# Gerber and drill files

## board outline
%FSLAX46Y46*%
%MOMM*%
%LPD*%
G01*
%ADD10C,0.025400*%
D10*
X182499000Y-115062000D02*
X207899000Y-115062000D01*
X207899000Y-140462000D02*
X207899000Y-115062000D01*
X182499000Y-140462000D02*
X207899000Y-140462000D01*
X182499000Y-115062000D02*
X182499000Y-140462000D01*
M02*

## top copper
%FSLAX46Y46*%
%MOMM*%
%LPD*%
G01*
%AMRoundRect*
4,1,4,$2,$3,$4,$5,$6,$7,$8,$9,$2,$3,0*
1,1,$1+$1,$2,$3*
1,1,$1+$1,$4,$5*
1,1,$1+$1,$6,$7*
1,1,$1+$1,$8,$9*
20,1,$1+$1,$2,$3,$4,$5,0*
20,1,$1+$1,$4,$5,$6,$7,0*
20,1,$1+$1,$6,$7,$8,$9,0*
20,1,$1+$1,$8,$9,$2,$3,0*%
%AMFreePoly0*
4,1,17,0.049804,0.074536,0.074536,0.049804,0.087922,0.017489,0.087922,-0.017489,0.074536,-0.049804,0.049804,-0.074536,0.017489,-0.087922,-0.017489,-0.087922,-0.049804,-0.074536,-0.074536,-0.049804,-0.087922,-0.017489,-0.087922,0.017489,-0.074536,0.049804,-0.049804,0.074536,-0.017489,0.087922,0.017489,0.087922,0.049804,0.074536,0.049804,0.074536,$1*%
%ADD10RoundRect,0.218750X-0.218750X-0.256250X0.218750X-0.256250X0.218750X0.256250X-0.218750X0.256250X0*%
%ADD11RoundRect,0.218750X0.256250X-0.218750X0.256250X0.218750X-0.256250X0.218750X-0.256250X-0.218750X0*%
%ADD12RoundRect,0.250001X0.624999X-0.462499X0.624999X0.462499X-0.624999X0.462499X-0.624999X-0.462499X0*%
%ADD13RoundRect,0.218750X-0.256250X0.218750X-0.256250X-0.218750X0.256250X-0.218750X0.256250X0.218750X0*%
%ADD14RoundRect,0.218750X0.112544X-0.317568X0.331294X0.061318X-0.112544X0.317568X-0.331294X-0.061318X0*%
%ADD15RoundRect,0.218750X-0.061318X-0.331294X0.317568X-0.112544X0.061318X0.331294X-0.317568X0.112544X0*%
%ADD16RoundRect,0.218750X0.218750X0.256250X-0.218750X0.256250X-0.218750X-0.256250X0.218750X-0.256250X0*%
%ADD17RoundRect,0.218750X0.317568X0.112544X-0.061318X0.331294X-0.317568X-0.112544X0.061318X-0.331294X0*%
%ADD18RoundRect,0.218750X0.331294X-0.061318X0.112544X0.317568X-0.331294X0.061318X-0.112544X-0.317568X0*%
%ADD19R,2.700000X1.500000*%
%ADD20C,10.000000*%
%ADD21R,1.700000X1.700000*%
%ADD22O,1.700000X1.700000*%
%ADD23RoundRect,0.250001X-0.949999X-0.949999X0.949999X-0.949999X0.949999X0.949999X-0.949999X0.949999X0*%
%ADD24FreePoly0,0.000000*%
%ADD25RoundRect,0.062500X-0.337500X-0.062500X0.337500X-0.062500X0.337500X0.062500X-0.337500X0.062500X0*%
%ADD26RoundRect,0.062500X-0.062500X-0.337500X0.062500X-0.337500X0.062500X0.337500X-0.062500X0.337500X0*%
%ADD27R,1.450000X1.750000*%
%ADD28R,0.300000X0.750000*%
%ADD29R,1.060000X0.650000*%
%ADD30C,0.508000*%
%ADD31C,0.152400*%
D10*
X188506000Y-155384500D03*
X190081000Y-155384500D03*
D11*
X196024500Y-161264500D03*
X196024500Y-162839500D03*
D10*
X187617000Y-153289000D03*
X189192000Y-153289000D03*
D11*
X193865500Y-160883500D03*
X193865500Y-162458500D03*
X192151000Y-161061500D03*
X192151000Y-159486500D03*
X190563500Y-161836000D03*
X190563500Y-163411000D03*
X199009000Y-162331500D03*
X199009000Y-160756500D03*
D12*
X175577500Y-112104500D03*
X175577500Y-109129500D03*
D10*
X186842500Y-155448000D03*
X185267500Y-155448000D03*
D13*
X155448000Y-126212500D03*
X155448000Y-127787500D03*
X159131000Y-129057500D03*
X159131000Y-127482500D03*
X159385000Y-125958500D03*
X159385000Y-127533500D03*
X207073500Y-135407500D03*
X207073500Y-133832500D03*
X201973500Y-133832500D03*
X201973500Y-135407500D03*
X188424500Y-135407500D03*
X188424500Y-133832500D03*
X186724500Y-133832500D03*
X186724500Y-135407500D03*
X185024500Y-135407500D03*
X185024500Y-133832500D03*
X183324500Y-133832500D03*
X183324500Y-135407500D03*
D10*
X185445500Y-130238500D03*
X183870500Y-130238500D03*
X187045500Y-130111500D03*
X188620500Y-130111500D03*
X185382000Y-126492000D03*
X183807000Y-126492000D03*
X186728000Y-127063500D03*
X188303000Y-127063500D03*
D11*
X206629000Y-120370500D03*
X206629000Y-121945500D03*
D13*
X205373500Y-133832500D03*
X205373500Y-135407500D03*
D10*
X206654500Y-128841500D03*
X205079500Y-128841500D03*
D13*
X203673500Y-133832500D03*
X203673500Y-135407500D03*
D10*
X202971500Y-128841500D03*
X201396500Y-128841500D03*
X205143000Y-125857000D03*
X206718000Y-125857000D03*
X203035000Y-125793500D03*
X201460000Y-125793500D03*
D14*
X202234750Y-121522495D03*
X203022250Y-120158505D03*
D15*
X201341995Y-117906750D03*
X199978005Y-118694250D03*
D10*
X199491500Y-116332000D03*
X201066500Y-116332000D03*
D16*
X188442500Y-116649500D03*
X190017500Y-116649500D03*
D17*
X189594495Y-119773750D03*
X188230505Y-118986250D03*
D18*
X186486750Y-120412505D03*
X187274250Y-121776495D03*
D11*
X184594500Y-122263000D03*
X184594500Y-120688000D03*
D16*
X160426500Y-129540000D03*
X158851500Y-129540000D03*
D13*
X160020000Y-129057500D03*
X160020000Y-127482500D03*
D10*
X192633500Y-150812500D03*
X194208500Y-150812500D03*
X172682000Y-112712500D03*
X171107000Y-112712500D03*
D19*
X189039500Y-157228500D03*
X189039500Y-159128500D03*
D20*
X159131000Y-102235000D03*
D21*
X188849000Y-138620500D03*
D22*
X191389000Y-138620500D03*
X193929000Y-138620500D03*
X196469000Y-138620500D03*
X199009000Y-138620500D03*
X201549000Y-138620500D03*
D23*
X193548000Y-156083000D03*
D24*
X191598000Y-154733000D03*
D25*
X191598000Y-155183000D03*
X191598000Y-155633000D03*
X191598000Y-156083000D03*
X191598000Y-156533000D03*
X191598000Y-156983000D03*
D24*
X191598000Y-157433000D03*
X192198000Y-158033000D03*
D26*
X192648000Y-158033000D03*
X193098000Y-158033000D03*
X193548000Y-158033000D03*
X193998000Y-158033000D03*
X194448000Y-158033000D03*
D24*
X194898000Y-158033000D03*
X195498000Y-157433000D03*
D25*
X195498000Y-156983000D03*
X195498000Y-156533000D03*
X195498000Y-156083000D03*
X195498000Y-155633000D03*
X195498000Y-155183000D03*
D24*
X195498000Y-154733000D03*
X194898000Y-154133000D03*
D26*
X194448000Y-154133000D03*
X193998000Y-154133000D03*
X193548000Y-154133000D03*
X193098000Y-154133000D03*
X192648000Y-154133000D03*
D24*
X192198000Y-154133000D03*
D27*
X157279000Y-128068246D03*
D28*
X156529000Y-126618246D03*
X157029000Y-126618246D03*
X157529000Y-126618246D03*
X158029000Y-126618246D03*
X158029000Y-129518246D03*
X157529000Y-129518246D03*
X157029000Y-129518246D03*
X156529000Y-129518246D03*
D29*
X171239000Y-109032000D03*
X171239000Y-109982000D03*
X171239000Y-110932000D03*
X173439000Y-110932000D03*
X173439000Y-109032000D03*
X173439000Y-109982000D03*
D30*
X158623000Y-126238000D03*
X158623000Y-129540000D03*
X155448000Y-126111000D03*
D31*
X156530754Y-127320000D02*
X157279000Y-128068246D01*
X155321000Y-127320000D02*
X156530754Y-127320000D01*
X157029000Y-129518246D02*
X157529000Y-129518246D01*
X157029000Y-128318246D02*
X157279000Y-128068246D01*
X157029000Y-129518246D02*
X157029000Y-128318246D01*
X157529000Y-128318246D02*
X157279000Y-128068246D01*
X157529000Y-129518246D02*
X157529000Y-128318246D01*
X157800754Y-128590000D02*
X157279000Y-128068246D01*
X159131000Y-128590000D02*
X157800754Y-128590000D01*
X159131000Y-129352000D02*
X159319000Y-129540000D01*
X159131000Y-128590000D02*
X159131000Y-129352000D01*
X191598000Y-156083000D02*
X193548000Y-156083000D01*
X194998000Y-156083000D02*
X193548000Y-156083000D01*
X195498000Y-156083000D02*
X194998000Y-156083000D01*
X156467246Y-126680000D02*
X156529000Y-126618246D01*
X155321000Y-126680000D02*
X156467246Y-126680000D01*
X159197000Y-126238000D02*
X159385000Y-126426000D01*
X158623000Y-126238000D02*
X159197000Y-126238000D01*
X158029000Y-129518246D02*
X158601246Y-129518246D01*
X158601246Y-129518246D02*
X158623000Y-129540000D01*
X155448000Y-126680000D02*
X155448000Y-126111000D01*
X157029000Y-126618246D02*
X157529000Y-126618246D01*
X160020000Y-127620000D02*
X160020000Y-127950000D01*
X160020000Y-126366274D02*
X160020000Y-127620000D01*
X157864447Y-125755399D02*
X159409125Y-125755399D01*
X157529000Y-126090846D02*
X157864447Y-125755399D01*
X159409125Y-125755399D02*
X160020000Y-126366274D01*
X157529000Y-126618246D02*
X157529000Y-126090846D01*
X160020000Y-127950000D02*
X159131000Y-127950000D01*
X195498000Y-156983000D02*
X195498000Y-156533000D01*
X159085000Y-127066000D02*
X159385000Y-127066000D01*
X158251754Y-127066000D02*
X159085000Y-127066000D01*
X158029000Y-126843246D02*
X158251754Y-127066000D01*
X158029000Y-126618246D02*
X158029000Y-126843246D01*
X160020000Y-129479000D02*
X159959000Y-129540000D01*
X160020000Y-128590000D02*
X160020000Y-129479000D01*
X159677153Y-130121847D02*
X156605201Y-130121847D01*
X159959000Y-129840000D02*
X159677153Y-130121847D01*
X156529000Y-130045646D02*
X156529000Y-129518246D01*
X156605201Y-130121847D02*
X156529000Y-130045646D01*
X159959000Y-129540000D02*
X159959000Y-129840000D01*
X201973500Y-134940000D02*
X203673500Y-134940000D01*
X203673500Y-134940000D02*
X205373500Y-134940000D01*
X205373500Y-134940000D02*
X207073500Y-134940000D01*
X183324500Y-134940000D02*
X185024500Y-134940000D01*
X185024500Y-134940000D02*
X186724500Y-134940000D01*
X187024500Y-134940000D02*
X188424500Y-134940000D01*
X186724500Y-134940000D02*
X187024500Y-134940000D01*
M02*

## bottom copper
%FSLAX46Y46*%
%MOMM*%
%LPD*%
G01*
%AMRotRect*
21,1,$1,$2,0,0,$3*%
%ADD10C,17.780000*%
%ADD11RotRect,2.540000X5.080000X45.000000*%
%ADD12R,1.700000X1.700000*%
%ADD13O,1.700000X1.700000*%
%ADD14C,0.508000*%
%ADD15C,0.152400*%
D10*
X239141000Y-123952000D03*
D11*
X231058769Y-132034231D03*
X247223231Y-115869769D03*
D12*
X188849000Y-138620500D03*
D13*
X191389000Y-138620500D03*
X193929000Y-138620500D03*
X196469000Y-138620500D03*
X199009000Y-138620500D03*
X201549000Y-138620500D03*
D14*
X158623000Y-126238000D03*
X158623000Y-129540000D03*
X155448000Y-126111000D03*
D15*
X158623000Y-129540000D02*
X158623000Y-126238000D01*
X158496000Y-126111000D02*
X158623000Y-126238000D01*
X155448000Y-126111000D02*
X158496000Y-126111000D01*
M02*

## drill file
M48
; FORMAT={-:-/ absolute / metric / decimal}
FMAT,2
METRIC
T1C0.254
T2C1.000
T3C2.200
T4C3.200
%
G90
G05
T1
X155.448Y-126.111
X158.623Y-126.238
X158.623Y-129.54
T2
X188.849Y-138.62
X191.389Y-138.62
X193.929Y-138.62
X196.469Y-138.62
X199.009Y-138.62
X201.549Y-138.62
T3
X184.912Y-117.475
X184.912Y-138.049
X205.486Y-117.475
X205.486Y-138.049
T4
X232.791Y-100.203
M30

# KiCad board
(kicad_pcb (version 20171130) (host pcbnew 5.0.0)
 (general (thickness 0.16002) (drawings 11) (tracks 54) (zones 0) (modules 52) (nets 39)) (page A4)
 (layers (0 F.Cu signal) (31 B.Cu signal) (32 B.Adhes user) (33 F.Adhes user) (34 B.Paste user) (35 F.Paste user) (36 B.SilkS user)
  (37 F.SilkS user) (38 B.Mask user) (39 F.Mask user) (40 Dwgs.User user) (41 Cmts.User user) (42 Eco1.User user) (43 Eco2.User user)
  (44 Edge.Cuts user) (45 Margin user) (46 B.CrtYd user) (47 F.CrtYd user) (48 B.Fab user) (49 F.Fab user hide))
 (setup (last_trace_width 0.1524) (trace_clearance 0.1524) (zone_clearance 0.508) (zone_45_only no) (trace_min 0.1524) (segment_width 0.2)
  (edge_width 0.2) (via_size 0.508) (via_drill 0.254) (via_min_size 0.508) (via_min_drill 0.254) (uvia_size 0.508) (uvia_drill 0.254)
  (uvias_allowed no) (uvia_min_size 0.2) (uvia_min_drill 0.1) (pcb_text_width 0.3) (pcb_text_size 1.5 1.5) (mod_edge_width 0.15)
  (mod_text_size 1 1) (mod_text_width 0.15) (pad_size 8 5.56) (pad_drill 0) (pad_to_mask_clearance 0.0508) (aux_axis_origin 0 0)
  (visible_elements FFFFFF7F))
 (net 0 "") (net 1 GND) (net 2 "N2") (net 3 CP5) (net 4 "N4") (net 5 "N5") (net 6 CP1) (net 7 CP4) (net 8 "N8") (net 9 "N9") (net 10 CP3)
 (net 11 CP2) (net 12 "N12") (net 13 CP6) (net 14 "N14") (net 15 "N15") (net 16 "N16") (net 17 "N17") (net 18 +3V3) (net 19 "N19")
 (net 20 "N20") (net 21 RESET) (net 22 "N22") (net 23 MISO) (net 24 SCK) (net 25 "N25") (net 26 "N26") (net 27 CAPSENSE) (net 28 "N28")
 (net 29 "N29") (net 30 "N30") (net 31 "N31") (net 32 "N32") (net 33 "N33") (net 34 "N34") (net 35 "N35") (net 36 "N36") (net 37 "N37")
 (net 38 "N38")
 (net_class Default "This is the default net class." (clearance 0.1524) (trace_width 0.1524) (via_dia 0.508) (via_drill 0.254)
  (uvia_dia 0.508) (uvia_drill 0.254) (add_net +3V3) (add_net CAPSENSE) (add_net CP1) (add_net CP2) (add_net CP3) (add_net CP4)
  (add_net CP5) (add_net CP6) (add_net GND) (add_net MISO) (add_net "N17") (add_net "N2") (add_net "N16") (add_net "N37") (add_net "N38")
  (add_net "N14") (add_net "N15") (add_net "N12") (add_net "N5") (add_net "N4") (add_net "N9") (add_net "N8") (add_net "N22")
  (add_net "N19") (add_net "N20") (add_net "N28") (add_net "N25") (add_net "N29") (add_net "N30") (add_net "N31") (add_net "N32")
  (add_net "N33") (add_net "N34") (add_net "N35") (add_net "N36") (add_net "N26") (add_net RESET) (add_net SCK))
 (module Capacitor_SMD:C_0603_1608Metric (layer F.Cu) (at 189.2935 155.3845)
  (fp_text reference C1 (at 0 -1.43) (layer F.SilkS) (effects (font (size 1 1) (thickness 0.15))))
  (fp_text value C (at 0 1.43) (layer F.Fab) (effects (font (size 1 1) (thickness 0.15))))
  (pad 1 smd roundrect (at -0.7875 0) (size 0.875 0.95) (layers F.Cu F.Paste F.Mask) (roundrect_rratio 0.25) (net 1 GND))
  (pad 2 smd roundrect (at 0.7875 0) (size 0.875 0.95) (layers F.Cu F.Paste F.Mask) (roundrect_rratio 0.25) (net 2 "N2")))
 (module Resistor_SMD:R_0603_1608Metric (layer F.Cu) (at 196.0245 162.052 90)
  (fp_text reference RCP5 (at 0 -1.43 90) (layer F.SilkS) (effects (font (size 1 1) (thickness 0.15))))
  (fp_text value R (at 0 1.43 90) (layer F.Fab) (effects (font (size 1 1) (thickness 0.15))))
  (pad 2 smd roundrect (at 0.7875 0 90) (size 0.875 0.95) (layers F.Cu F.Paste F.Mask) (roundrect_rratio 0.25) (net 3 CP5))
  (pad 1 smd roundrect (at -0.7875 0 90) (size 0.875 0.95) (layers F.Cu F.Paste F.Mask) (roundrect_rratio 0.25) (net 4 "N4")))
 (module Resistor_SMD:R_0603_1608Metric (layer F.Cu) (at 188.4045 153.289)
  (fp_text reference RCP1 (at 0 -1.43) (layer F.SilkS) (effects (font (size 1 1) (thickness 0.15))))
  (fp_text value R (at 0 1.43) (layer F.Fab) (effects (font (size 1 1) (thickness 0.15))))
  (pad 1 smd roundrect (at -0.7875 0) (size 0.875 0.95) (layers F.Cu F.Paste F.Mask) (roundrect_rratio 0.25) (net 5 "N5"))
  (pad 2 smd roundrect (at 0.7875 0) (size 0.875 0.95) (layers F.Cu F.Paste F.Mask) (roundrect_rratio 0.25) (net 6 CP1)))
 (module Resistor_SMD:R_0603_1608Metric (layer F.Cu) (at 193.8655 161.671 90)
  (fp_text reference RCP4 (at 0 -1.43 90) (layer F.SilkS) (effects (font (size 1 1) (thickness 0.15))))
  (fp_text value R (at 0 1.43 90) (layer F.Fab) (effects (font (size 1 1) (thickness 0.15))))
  (pad 2 smd roundrect (at 0.7875 0 90) (size 0.875 0.95) (layers F.Cu F.Paste F.Mask) (roundrect_rratio 0.25) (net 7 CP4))
  (pad 1 smd roundrect (at -0.7875 0 90) (size 0.875 0.95) (layers F.Cu F.Paste F.Mask) (roundrect_rratio 0.25) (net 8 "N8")))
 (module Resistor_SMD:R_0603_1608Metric (layer F.Cu) (at 192.151 160.274 90)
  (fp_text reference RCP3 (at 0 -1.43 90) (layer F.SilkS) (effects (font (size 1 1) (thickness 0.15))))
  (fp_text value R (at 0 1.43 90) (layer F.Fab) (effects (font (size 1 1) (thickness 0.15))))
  (pad 1 smd roundrect (at -0.7875 0 90) (size 0.875 0.95) (layers F.Cu F.Paste F.Mask) (roundrect_rratio 0.25) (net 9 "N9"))
  (pad 2 smd roundrect (at 0.7875 0 90) (size 0.875 0.95) (layers F.Cu F.Paste F.Mask) (roundrect_rratio 0.25) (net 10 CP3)))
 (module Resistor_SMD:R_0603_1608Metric (layer F.Cu) (at 190.5635 162.6235 90)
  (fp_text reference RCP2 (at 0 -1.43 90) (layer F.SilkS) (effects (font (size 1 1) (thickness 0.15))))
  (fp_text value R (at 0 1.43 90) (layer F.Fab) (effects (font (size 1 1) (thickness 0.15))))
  (pad 2 smd roundrect (at 0.7875 0 90) (size 0.875 0.95) (layers F.Cu F.Paste F.Mask) (roundrect_rratio 0.25) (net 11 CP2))
  (pad 1 smd roundrect (at -0.7875 0 90) (size 0.875 0.95) (layers F.Cu F.Paste F.Mask) (roundrect_rratio 0.25) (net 5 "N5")))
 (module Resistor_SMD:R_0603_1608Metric (layer F.Cu) (at 199.009 161.544 90)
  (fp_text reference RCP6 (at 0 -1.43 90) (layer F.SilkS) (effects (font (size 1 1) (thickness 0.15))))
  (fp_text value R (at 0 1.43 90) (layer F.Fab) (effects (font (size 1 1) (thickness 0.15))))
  (pad 1 smd roundrect (at -0.7875 0 90) (size 0.875 0.95) (layers F.Cu F.Paste F.Mask) (roundrect_rratio 0.25) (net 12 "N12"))
  (pad 2 smd roundrect (at 0.7875 0 90) (size 0.875 0.95) (layers F.Cu F.Paste F.Mask) (roundrect_rratio 0.25) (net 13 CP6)))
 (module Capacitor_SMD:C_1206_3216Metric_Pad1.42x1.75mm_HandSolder (layer F.Cu) (at 175.5775 110.617 90)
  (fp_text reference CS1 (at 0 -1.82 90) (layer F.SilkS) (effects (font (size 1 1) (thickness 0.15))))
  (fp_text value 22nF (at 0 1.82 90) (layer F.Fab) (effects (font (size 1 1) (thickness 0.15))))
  (pad 1 smd roundrect (at -1.4875 0 90) (size 1.425 1.75) (layers F.Cu F.Paste F.Mask) (roundrect_rratio 0.175439) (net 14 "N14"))
  (pad 2 smd roundrect (at 1.4875 0 90) (size 1.425 1.75) (layers F.Cu F.Paste F.Mask) (roundrect_rratio 0.175439) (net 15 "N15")))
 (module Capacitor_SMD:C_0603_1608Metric (layer F.Cu) (at 186.055 155.448)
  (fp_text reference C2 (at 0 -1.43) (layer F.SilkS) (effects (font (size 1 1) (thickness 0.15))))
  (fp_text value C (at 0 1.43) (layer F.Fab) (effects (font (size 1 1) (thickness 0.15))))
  (pad 2 smd roundrect (at 0.7875 0) (size 0.875 0.95) (layers F.Cu F.Paste F.Mask) (roundrect_rratio 0.25) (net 1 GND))
  (pad 1 smd roundrect (at -0.7875 0) (size 0.875 0.95) (layers F.Cu F.Paste F.Mask) (roundrect_rratio 0.25) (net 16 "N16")))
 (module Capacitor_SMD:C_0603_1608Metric (layer F.Cu) (at 155.448 127 270)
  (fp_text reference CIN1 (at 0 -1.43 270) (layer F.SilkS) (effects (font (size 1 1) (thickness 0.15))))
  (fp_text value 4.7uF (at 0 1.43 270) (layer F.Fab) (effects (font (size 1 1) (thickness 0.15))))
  (pad 1 smd roundrect (at -0.7875 0 270) (size 0.875 0.95) (layers F.Cu F.Paste F.Mask) (roundrect_rratio 0.25) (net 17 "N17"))
  (pad 2 smd roundrect (at 0.7875 0 270) (size 0.875 0.95) (layers F.Cu F.Paste F.Mask) (roundrect_rratio 0.25) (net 1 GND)))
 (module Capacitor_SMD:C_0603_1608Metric (layer F.Cu) (at 159.131 128.27 270)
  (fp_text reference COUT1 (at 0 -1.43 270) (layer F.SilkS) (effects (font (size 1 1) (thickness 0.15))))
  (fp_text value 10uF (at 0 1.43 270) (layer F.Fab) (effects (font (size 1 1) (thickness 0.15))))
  (pad 2 smd roundrect (at 0.7875 0 270) (size 0.875 0.95) (layers F.Cu F.Paste F.Mask) (roundrect_rratio 0.25) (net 1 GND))
  (pad 1 smd roundrect (at -0.7875 0 270) (size 0.875 0.95) (layers F.Cu F.Paste F.Mask) (roundrect_rratio 0.25) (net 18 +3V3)))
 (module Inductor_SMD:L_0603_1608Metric (layer F.Cu) (at 159.385 126.746 270)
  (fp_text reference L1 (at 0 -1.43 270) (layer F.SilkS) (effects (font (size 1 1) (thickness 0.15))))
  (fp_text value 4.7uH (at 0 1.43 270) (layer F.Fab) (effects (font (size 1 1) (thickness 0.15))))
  (pad 1 smd roundrect (at -0.7875 0 270) (size 0.875 0.95) (layers F.Cu F.Paste F.Mask) (roundrect_rratio 0.25) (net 17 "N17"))
  (pad 2 smd roundrect (at 0.7875 0 270) (size 0.875 0.95) (layers F.Cu F.Paste F.Mask) (roundrect_rratio 0.25) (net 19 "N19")))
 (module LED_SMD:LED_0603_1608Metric (layer F.Cu) (at 207.0735 134.62 270)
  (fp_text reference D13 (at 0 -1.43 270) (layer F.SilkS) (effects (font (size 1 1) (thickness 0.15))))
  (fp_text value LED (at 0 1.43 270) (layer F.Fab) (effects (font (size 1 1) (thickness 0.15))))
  (pad 2 smd roundrect (at 0.7875 0 270) (size 0.875 0.95) (layers F.Cu F.Paste F.Mask) (roundrect_rratio 0.25) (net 8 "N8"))
  (pad 1 smd roundrect (at -0.7875 0 270) (size 0.875 0.95) (layers F.Cu F.Paste F.Mask) (roundrect_rratio 0.25) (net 12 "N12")))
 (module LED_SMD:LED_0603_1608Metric (layer F.Cu) (at 201.9735 134.62 270)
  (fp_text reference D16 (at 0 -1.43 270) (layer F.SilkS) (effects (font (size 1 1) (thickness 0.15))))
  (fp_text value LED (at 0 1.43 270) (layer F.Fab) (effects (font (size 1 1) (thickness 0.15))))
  (pad 1 smd roundrect (at -0.7875 0 270) (size 0.875 0.95) (layers F.Cu F.Paste F.Mask) (roundrect_rratio 0.25) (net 5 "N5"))
  (pad 2 smd roundrect (at 0.7875 0 270) (size 0.875 0.95) (layers F.Cu F.Paste F.Mask) (roundrect_rratio 0.25) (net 8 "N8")))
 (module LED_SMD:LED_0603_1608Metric (layer F.Cu) (at 188.4245 134.62 270)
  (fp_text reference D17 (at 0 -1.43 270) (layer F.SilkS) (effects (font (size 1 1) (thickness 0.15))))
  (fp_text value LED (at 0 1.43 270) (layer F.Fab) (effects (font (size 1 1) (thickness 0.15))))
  (pad 2 smd roundrect (at 0.7875 0 270) (size 0.875 0.95) (layers F.Cu F.Paste F.Mask) (roundrect_rratio 0.25) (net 4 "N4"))
  (pad 1 smd roundrect (at -0.7875 0 270) (size 0.875 0.95) (layers F.Cu F.Paste F.Mask) (roundrect_rratio 0.25) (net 12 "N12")))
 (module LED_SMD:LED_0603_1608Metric (layer F.Cu) (at 186.7245 134.62 270)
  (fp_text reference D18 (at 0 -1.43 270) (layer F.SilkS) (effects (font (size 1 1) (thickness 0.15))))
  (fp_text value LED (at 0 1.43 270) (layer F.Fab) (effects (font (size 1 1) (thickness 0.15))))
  (pad 1 smd roundrect (at -0.7875 0 270) (size 0.875 0.95) (layers F.Cu F.Paste F.Mask) (roundrect_rratio 0.25) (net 8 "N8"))
  (pad 2 smd roundrect (at 0.7875 0 270) (size 0.875 0.95) (layers F.Cu F.Paste F.Mask) (roundrect_rratio 0.25) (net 4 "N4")))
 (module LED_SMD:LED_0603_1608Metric (layer F.Cu) (at 185.0245 134.62 270)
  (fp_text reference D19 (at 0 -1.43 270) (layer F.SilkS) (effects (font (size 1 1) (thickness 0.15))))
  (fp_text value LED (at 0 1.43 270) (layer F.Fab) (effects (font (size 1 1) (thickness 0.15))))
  (pad 2 smd roundrect (at 0.7875 0 270) (size 0.875 0.95) (layers F.Cu F.Paste F.Mask) (roundrect_rratio 0.25) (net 4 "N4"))
  (pad 1 smd roundrect (at -0.7875 0 270) (size 0.875 0.95) (layers F.Cu F.Paste F.Mask) (roundrect_rratio 0.25) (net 9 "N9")))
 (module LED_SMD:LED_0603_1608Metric (layer F.Cu) (at 183.3245 134.62 270)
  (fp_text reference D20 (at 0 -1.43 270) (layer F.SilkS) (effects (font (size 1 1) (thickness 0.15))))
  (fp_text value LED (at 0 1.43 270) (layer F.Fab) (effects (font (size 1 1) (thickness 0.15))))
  (pad 1 smd roundrect (at -0.7875 0 270) (size 0.875 0.95) (layers F.Cu F.Paste F.Mask) (roundrect_rratio 0.25) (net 5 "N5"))
  (pad 2 smd roundrect (at 0.7875 0 270) (size 0.875 0.95) (layers F.Cu F.Paste F.Mask) (roundrect_rratio 0.25) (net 4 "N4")))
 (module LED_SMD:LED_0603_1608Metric (layer F.Cu) (at 184.658 130.2385)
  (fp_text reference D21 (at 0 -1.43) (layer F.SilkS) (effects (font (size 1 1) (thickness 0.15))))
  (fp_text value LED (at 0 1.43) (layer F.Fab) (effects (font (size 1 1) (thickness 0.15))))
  (pad 2 smd roundrect (at 0.7875 0) (size 0.875 0.95) (layers F.Cu F.Paste F.Mask) (roundrect_rratio 0.25) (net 12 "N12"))
  (pad 1 smd roundrect (at -0.7875 0) (size 0.875 0.95) (layers F.Cu F.Paste F.Mask) (roundrect_rratio 0.25) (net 4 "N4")))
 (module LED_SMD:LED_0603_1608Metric (layer F.Cu) (at 187.833 130.1115)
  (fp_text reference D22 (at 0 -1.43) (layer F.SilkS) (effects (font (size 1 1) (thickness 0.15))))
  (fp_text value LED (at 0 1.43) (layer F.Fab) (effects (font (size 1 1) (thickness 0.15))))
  (pad 1 smd roundrect (at -0.7875 0) (size 0.875 0.95) (layers F.Cu F.Paste F.Mask) (roundrect_rratio 0.25) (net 8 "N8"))
  (pad 2 smd roundrect (at 0.7875 0) (size 0.875 0.95) (layers F.Cu F.Paste F.Mask) (roundrect_rratio 0.25) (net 12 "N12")))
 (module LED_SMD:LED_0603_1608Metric (layer F.Cu) (at 184.5945 126.492)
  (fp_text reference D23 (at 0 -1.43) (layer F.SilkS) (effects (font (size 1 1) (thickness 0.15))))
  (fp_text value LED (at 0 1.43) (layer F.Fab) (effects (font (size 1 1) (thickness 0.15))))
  (pad 2 smd roundrect (at 0.7875 0) (size 0.875 0.95) (layers F.Cu F.Paste F.Mask) (roundrect_rratio 0.25) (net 12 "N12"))
  (pad 1 smd roundrect (at -0.7875 0) (size 0.875 0.95) (layers F.Cu F.Paste F.Mask) (roundrect_rratio 0.25) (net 9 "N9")))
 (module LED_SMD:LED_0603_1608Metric (layer F.Cu) (at 187.5155 127.0635)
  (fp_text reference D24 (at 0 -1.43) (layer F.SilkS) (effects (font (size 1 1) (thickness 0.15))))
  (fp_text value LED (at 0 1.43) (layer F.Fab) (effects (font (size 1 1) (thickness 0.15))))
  (pad 1 smd roundrect (at -0.7875 0) (size 0.875 0.95) (layers F.Cu F.Paste F.Mask) (roundrect_rratio 0.25) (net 5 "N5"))
  (pad 2 smd roundrect (at 0.7875 0) (size 0.875 0.95) (layers F.Cu F.Paste F.Mask) (roundrect_rratio 0.25) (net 12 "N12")))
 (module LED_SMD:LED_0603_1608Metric (layer F.Cu) (at 206.629 121.158 90)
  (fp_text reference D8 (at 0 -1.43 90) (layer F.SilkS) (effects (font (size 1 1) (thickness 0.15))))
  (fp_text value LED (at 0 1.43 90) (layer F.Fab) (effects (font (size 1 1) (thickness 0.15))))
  (pad 2 smd roundrect (at 0.7875 0 90) (size 0.875 0.95) (layers F.Cu F.Paste F.Mask) (roundrect_rratio 0.25) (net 5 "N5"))
  (pad 1 smd roundrect (at -0.7875 0 90) (size 0.875 0.95) (layers F.Cu F.Paste F.Mask) (roundrect_rratio 0.25) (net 9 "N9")))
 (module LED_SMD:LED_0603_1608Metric (layer F.Cu) (at 205.3735 134.62 270)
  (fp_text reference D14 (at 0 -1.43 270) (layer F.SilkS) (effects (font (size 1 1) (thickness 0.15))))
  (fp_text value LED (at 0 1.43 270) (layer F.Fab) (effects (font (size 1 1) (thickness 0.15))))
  (pad 1 smd roundrect (at -0.7875 0 270) (size 0.875 0.95) (layers F.Cu F.Paste F.Mask) (roundrect_rratio 0.25) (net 4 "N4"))
  (pad 2 smd roundrect (at 0.7875 0 270) (size 0.875 0.95) (layers F.Cu F.Paste F.Mask) (roundrect_rratio 0.25) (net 8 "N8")))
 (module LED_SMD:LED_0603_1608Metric (layer F.Cu) (at 205.867 128.8415)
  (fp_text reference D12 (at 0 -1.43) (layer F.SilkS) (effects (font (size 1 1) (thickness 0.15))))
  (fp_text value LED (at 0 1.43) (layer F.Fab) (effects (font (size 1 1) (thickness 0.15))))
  (pad 2 smd roundrect (at 0.7875 0) (size 0.875 0.95) (layers F.Cu F.Paste F.Mask) (roundrect_rratio 0.25) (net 9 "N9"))
  (pad 1 smd roundrect (at -0.7875 0) (size 0.875 0.95) (layers F.Cu F.Paste F.Mask) (roundrect_rratio 0.25) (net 5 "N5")))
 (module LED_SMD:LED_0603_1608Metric (layer F.Cu) (at 203.6735 134.62 270)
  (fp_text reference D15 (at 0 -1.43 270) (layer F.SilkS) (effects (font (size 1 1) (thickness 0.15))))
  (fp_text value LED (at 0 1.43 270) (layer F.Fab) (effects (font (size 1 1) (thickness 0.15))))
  (pad 1 smd roundrect (at -0.7875 0 270) (size 0.875 0.95) (layers F.Cu F.Paste F.Mask) (roundrect_rratio 0.25) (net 9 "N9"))
  (pad 2 smd roundrect (at 0.7875 0 270) (size 0.875 0.95) (layers F.Cu F.Paste F.Mask) (roundrect_rratio 0.25) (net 8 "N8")))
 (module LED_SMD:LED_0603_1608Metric (layer F.Cu) (at 202.184 128.8415)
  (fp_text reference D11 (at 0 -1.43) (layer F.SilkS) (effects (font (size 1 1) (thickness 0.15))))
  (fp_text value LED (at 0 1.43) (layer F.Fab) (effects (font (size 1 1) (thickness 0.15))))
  (pad 2 smd roundrect (at 0.7875 0) (size 0.875 0.95) (layers F.Cu F.Paste F.Mask) (roundrect_rratio 0.25) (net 9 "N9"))
  (pad 1 smd roundrect (at -0.7875 0) (size 0.875 0.95) (layers F.Cu F.Paste F.Mask) (roundrect_rratio 0.25) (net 8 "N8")))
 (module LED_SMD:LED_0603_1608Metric (layer F.Cu) (at 205.9305 125.857)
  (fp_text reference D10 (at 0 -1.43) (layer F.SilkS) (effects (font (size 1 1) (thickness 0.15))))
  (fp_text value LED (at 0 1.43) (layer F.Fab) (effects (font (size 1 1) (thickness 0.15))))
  (pad 1 smd roundrect (at -0.7875 0) (size 0.875 0.95) (layers F.Cu F.Paste F.Mask) (roundrect_rratio 0.25) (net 4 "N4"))
  (pad 2 smd roundrect (at 0.7875 0) (size 0.875 0.95) (layers F.Cu F.Paste F.Mask) (roundrect_rratio 0.25) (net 9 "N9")))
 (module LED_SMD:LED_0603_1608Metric (layer F.Cu) (at 202.2475 125.7935)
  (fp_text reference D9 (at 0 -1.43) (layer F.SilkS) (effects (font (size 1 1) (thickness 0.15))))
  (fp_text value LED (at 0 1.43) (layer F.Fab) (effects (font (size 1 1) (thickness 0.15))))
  (pad 2 smd roundrect (at 0.7875 0) (size 0.875 0.95) (layers F.Cu F.Paste F.Mask) (roundrect_rratio 0.25) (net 9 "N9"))
  (pad 1 smd roundrect (at -0.7875 0) (size 0.875 0.95) (layers F.Cu F.Paste F.Mask) (roundrect_rratio 0.25) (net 12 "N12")))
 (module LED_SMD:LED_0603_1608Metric (layer F.Cu) (at 202.6285 120.8405 60)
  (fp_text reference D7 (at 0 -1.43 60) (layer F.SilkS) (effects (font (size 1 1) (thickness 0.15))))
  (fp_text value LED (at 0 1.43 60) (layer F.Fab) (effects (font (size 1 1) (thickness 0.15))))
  (pad 1 smd roundrect (at -0.7875 0 60) (size 0.875 0.95) (layers F.Cu F.Paste F.Mask) (roundrect_rratio 0.25) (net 8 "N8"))
  (pad 2 smd roundrect (at 0.7875 0 60) (size 0.875 0.95) (layers F.Cu F.Paste F.Mask) (roundrect_rratio 0.25) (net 5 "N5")))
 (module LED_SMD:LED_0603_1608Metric (layer F.Cu) (at 200.66 118.3005 30)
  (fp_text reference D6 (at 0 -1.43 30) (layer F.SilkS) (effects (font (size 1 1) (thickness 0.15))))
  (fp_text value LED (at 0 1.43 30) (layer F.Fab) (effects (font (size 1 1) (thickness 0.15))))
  (pad 2 smd roundrect (at 0.7875 0 30) (size 0.875 0.95) (layers F.Cu F.Paste F.Mask) (roundrect_rratio 0.25) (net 5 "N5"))
  (pad 1 smd roundrect (at -0.7875 0 30) (size 0.875 0.95) (layers F.Cu F.Paste F.Mask) (roundrect_rratio 0.25) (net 4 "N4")))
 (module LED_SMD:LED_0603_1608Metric (layer F.Cu) (at 200.279 116.332)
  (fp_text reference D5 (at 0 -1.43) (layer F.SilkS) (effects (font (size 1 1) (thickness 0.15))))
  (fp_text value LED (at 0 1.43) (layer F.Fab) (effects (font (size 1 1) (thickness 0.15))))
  (pad 1 smd roundrect (at -0.7875 0) (size 0.875 0.95) (layers F.Cu F.Paste F.Mask) (roundrect_rratio 0.25) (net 12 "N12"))
  (pad 2 smd roundrect (at 0.7875 0) (size 0.875 0.95) (layers F.Cu F.Paste F.Mask) (roundrect_rratio 0.25) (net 5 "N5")))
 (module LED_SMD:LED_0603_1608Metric (layer F.Cu) (at 189.23 116.6495 180)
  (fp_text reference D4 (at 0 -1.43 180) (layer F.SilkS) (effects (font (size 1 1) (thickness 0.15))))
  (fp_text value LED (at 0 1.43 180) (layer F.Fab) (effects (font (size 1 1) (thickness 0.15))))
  (pad 2 smd roundrect (at 0.7875 0 180) (size 0.875 0.95) (layers F.Cu F.Paste F.Mask) (roundrect_rratio 0.25) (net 5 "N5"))
  (pad 1 smd roundrect (at -0.7875 0 180) (size 0.875 0.95) (layers F.Cu F.Paste F.Mask) (roundrect_rratio 0.25) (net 9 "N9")))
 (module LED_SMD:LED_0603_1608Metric (layer F.Cu) (at 188.9125 119.38 150)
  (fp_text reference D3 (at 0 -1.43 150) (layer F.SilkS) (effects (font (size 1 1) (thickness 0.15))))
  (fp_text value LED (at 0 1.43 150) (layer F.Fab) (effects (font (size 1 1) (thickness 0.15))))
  (pad 1 smd roundrect (at -0.7875 0 150) (size 0.875 0.95) (layers F.Cu F.Paste F.Mask) (roundrect_rratio 0.25) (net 8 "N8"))
  (pad 2 smd roundrect (at 0.7875 0 150) (size 0.875 0.95) (layers F.Cu F.Paste F.Mask) (roundrect_rratio 0.25) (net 5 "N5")))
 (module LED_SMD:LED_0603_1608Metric (layer F.Cu) (at 186.8805 121.0945 120)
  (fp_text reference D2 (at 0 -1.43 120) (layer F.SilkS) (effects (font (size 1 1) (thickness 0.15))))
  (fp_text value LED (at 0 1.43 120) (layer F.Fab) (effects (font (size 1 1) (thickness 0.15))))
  (pad 2 smd roundrect (at 0.7875 0 120) (size 0.875 0.95) (layers F.Cu F.Paste F.Mask) (roundrect_rratio 0.25) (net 5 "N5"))
  (pad 1 smd roundrect (at -0.7875 0 120) (size 0.875 0.95) (layers F.Cu F.Paste F.Mask) (roundrect_rratio 0.25) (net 4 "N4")))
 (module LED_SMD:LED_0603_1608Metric (layer F.Cu) (at 184.5945 121.4755 90)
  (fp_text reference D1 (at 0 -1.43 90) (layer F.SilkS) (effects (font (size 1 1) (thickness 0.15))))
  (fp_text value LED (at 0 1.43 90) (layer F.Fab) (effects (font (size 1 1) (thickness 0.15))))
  (pad 1 smd roundrect (at -0.7875 0 90) (size 0.875 0.95) (layers F.Cu F.Paste F.Mask) (roundrect_rratio 0.25) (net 12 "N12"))
  (pad 2 smd roundrect (at 0.7875 0 90) (size 0.875 0.95) (layers F.Cu F.Paste F.Mask) (roundrect_rratio 0.25) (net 5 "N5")))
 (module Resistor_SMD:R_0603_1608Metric (layer F.Cu) (at 159.639 129.54 180)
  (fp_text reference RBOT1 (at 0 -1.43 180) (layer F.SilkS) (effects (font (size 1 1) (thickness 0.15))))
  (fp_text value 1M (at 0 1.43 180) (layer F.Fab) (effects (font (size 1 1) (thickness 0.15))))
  (pad 1 smd roundrect (at -0.7875 0 180) (size 0.875 0.95) (layers F.Cu F.Paste F.Mask) (roundrect_rratio 0.25) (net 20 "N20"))
  (pad 2 smd roundrect (at 0.7875 0 180) (size 0.875 0.95) (layers F.Cu F.Paste F.Mask) (roundrect_rratio 0.25) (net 1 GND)))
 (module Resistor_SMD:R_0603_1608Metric (layer F.Cu) (at 160.02 128.27 270)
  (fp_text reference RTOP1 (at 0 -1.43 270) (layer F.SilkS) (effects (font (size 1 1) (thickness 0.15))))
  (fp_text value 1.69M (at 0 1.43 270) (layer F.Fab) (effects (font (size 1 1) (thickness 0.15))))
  (pad 2 smd roundrect (at 0.7875 0 270) (size 0.875 0.95) (layers F.Cu F.Paste F.Mask) (roundrect_rratio 0.25) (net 20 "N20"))
  (pad 1 smd roundrect (at -0.7875 0 270) (size 0.875 0.95) (layers F.Cu F.Paste F.Mask) (roundrect_rratio 0.25) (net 18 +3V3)))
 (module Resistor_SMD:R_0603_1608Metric (layer F.Cu) (at 193.421 150.8125)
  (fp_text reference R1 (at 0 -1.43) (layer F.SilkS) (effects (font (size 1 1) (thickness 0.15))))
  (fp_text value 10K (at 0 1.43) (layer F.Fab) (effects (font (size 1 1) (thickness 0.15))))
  (pad 1 smd roundrect (at -0.7875 0) (size 0.875 0.95) (layers F.Cu F.Paste F.Mask) (roundrect_rratio 0.25) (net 18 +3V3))
  (pad 2 smd roundrect (at 0.7875 0) (size 0.875 0.95) (layers F.Cu F.Paste F.Mask) (roundrect_rratio 0.25) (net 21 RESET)))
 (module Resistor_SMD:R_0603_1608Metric (layer F.Cu) (at 171.8945 112.7125)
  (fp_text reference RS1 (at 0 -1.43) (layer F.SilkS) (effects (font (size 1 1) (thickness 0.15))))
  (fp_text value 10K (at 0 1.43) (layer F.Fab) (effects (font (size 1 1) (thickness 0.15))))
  (pad 2 smd roundrect (at 0.7875 0) (size 0.875 0.95) (layers F.Cu F.Paste F.Mask) (roundrect_rratio 0.25) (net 14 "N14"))
  (pad 1 smd roundrect (at -0.7875 0) (size 0.875 0.95) (layers F.Cu F.Paste F.Mask) (roundrect_rratio 0.25) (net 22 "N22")))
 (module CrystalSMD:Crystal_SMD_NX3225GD (layer F.Cu) (at 189.0395 158.1785 90)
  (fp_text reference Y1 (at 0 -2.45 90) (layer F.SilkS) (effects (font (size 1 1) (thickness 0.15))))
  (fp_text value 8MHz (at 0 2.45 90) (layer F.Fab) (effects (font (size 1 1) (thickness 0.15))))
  (pad 2 smd rect (at 0.95 0 90) (size 1.5 2.7) (layers F.Cu F.Paste F.Mask) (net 2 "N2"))
  (pad 1 smd rect (at -0.95 0 90) (size 1.5 2.7) (layers F.Cu F.Paste F.Mask) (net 16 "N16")))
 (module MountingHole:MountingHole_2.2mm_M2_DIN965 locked (layer F.Cu) (at 205.486 138.049)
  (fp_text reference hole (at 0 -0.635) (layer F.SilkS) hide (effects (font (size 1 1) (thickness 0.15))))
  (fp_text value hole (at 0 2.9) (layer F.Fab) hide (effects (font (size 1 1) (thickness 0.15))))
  (pad 1 np_thru_hole circle (at 0 0) (size 2.2 2.2) (drill 2.2) (layers *.Cu *.Mask)))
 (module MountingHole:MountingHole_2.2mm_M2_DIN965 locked (layer F.Cu) (at 184.912 117.475)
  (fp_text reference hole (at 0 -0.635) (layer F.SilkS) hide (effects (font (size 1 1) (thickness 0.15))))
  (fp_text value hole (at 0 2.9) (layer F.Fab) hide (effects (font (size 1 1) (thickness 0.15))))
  (pad 1 np_thru_hole circle (at 0 0) (size 2.2 2.2) (drill 2.2) (layers *.Cu *.Mask)))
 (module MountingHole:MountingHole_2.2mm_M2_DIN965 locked (layer F.Cu) (at 184.912 138.049)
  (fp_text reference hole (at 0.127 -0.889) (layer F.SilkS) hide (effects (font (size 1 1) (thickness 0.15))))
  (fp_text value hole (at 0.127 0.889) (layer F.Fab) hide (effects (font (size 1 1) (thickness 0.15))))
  (pad 1 np_thru_hole circle (at 0 0) (size 2.2 2.2) (drill 2.2) (layers *.Cu *.Mask)))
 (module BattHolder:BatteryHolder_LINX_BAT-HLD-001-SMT (layer B.Cu) (at 239.141 123.952 45)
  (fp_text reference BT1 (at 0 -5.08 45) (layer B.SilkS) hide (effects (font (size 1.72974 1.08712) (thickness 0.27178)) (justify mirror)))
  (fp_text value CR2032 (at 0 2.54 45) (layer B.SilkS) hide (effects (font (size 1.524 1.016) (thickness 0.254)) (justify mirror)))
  (pad 2 smd circle (at 0 0 45) (size 17.78 17.78) (layers B.Cu B.Paste B.Mask) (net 1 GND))
  (pad 1 smd rect (at -11.430001 0 45) (size 2.54 5.08) (layers B.Cu B.Paste B.Mask) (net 17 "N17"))
  (pad 1 smd rect (at 11.430001 0 45) (size 2.54 5.08) (layers B.Cu B.Paste B.Mask) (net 17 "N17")))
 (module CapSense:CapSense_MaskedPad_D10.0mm (layer F.Cu) (at 159.131 102.235)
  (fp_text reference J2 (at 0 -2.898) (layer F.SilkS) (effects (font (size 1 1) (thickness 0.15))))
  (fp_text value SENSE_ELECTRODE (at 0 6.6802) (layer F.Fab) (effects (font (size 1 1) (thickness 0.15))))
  (pad 1 smd circle (at 0 0) (size 10 10) (layers F.Cu) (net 22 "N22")))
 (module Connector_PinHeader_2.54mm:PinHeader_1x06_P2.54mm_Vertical (layer F.Cu) (at 188.849 138.6205 90)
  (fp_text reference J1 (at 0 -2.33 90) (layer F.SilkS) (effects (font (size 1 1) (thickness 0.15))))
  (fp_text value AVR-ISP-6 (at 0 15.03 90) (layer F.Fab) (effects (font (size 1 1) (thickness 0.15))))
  (pad 1 thru_hole rect (at 0 0 90) (size 1.7 1.7) (drill 1) (layers *.Cu *.Mask) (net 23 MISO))
  (pad 2 thru_hole oval (at 0 2.54 90) (size 1.7 1.7) (drill 1) (layers *.Cu *.Mask) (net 18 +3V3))
  (pad 3 thru_hole oval (at 0 5.08 90) (size 1.7 1.7) (drill 1) (layers *.Cu *.Mask) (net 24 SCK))
  (pad 4 thru_hole oval (at 0 7.62 90) (size 1.7 1.7) (drill 1) (layers *.Cu *.Mask) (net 13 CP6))
  (pad 5 thru_hole oval (at 0 10.16 90) (size 1.7 1.7) (drill 1) (layers *.Cu *.Mask) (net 21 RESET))
  (pad 6 thru_hole oval (at 0 12.7 90) (size 1.7 1.7) (drill 1) (layers *.Cu *.Mask) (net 1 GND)))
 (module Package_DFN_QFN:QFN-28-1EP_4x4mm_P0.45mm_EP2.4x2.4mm (layer F.Cu) (at 193.548 156.083)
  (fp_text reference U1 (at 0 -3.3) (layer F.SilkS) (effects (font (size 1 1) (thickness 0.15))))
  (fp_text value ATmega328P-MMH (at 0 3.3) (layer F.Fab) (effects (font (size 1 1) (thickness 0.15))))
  (pad 29 smd roundrect (at 0 0) (size 2.4 2.4) (layers F.Cu F.Mask) (roundrect_rratio 0.104167) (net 1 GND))
  (pad "" smd roundrect (at -0.6 -0.6) (size 0.97 0.97) (layers F.Paste) (roundrect_rratio 0.25))
  (pad "" smd roundrect (at -0.6 0.6) (size 0.97 0.97) (layers F.Paste) (roundrect_rratio 0.25))
  (pad "" smd roundrect (at 0.6 -0.6) (size 0.97 0.97) (layers F.Paste) (roundrect_rratio 0.25))
  (pad "" smd roundrect (at 0.6 0.6) (size 0.97 0.97) (layers F.Paste) (roundrect_rratio 0.25))
  (pad 1 smd custom (at -1.95 -1.35) (size 0.179289 0.179289) (layers F.Cu F.Paste F.Mask) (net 6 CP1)
   (options (clearance outline) (anchor circle)) (primitives))
  (pad 2 smd roundrect (at -1.95 -0.9) (size 0.8 0.25) (layers F.Cu F.Paste F.Mask) (roundrect_rratio 0.25) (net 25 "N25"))
  (pad 3 smd roundrect (at -1.95 -0.45) (size 0.8 0.25) (layers F.Cu F.Paste F.Mask) (roundrect_rratio 0.25) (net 18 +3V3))
  (pad 4 smd roundrect (at -1.95 0) (size 0.8 0.25) (layers F.Cu F.Paste F.Mask) (roundrect_rratio 0.25) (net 1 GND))
  (pad 5 smd roundrect (at -1.95 0.45) (size 0.8 0.25) (layers F.Cu F.Paste F.Mask) (roundrect_rratio 0.25) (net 2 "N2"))
  (pad 6 smd roundrect (at -1.95 0.9) (size 0.8 0.25) (layers F.Cu F.Paste F.Mask) (roundrect_rratio 0.25) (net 16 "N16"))
  (pad 7 smd custom (at -1.95 1.35) (size 0.179289 0.179289) (layers F.Cu F.Paste F.Mask) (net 11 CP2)
   (options (clearance outline) (anchor circle)) (primitives))
  (pad 8 smd custom (at -1.35 1.95) (size 0.179289 0.179289) (layers F.Cu F.Paste F.Mask) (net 10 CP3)
   (options (clearance outline) (anchor circle)) (primitives))
  (pad 9 smd roundrect (at -0.9 1.95) (size 0.25 0.8) (layers F.Cu F.Paste F.Mask) (roundrect_rratio 0.25) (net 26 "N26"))
  (pad 10 smd roundrect (at -0.45 1.95) (size 0.25 0.8) (layers F.Cu F.Paste F.Mask) (roundrect_rratio 0.25) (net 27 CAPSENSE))
  (pad 11 smd roundrect (at 0 1.95) (size 0.25 0.8) (layers F.Cu F.Paste F.Mask) (roundrect_rratio 0.25) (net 7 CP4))
  (pad 12 smd roundrect (at 0.45 1.95) (size 0.25 0.8) (layers F.Cu F.Paste F.Mask) (roundrect_rratio 0.25) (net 3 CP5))
  (pad 13 smd roundrect (at 0.9 1.95) (size 0.25 0.8) (layers F.Cu F.Paste F.Mask) (roundrect_rratio 0.25) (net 13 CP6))
  (pad 14 smd custom (at 1.35 1.95) (size 0.179289 0.179289) (layers F.Cu F.Paste F.Mask) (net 23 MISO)
   (options (clearance outline) (anchor circle)) (primitives))
  (pad 15 smd custom (at 1.95 1.35) (size 0.179289 0.179289) (layers F.Cu F.Paste F.Mask) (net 24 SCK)
   (options (clearance outline) (anchor circle)) (primitives))
  (pad 16 smd roundrect (at 1.95 0.9) (size 0.8 0.25) (layers F.Cu F.Paste F.Mask) (roundrect_rratio 0.25) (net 18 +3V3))
  (pad 17 smd roundrect (at 1.95 0.45) (size 0.8 0.25) (layers F.Cu F.Paste F.Mask) (roundrect_rratio 0.25) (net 18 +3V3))
  (pad 18 smd roundrect (at 1.95 0) (size 0.8 0.25) (layers F.Cu F.Paste F.Mask) (roundrect_rratio 0.25) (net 1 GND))
  (pad 19 smd roundrect (at 1.95 -0.45) (size 0.8 0.25) (layers F.Cu F.Paste F.Mask) (roundrect_rratio 0.25) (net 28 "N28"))
  (pad 20 smd roundrect (at 1.95 -0.9) (size 0.8 0.25) (layers F.Cu F.Paste F.Mask) (roundrect_rratio 0.25) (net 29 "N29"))
  (pad 21 smd custom (at 1.95 -1.35) (size 0.179289 0.179289) (layers F.Cu F.Paste F.Mask) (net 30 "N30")
   (options (clearance outline) (anchor circle)) (primitives))
  (pad 22 smd custom (at 1.35 -1.95) (size 0.179289 0.179289) (layers F.Cu F.Paste F.Mask) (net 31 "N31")
   (options (clearance outline) (anchor circle)) (primitives))
  (pad 23 smd roundrect (at 0.9 -1.95) (size 0.25 0.8) (layers F.Cu F.Paste F.Mask) (roundrect_rratio 0.25) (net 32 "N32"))
  (pad 24 smd roundrect (at 0.45 -1.95) (size 0.25 0.8) (layers F.Cu F.Paste F.Mask) (roundrect_rratio 0.25) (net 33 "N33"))
  (pad 25 smd roundrect (at 0 -1.95) (size 0.25 0.8) (layers F.Cu F.Paste F.Mask) (roundrect_rratio 0.25) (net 21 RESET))
  (pad 26 smd roundrect (at -0.45 -1.95) (size 0.25 0.8) (layers F.Cu F.Paste F.Mask) (roundrect_rratio 0.25) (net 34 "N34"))
  (pad 27 smd roundrect (at -0.9 -1.95) (size 0.25 0.8) (layers F.Cu F.Paste F.Mask) (roundrect_rratio 0.25) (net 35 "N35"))
  (pad 28 smd custom (at -1.35 -1.95) (size 0.179289 0.179289) (layers F.Cu F.Paste F.Mask) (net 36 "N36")
   (options (clearance outline) (anchor circle)) (primitives)))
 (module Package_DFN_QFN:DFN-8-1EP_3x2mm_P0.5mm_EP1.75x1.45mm (layer F.Cu) (at 157.279 128.068246 90)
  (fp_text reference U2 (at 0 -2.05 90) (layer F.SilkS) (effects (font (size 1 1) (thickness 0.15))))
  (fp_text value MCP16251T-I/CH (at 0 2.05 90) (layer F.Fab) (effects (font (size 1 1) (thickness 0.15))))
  (pad "" smd rect (at -0.4375 -0.3625 90) (size 0.71 0.58) (layers F.Paste))
  (pad "" smd rect (at 0.4375 -0.3625 90) (size 0.71 0.58) (layers F.Paste))
  (pad "" smd rect (at 0.4375 0.3625 90) (size 0.71 0.58) (layers F.Paste))
  (pad 9 smd rect (at 0 0 90) (size 1.75 1.45) (layers F.Cu F.Mask) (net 1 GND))
  (pad "" smd rect (at -0.4375 0.3625 90) (size 0.71 0.58) (layers F.Paste))
  (pad 8 smd rect (at 1.45 -0.75 90) (size 0.75 0.3) (layers F.Cu F.Paste F.Mask) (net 17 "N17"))
  (pad 7 smd rect (at 1.45 -0.25 90) (size 0.75 0.3) (layers F.Cu F.Paste F.Mask) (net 18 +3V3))
  (pad 6 smd rect (at 1.45 0.25 90) (size 0.75 0.3) (layers F.Cu F.Paste F.Mask) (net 18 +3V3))
  (pad 5 smd rect (at 1.45 0.75 90) (size 0.75 0.3) (layers F.Cu F.Paste F.Mask) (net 19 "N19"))
  (pad 4 smd rect (at -1.45 0.75 90) (size 0.75 0.3) (layers F.Cu F.Paste F.Mask) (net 17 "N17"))
  (pad 3 smd rect (at -1.45 0.25 90) (size 0.75 0.3) (layers F.Cu F.Paste F.Mask) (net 1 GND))
  (pad 2 smd rect (at -1.45 -0.25 90) (size 0.75 0.3) (layers F.Cu F.Paste F.Mask) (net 1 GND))
  (pad 1 smd rect (at -1.45 -0.75 90) (size 0.75 0.3) (layers F.Cu F.Paste F.Mask) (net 20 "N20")))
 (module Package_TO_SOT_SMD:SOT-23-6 (layer F.Cu) (at 172.339 109.982)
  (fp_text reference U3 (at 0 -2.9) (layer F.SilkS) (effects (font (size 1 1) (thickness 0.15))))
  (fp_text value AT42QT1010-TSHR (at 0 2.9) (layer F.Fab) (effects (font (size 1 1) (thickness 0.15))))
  (pad 1 smd rect (at -1.1 -0.95) (size 1.06 0.65) (layers F.Cu F.Paste F.Mask) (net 27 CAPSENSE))
  (pad 2 smd rect (at -1.1 0) (size 1.06 0.65) (layers F.Cu F.Paste F.Mask) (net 1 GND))
  (pad 3 smd rect (at -1.1 0.95) (size 1.06 0.65) (layers F.Cu F.Paste F.Mask) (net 14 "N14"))
  (pad 4 smd rect (at 1.1 0.95) (size 1.06 0.65) (layers F.Cu F.Paste F.Mask) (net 15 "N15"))
  (pad 6 smd rect (at 1.1 -0.95) (size 1.06 0.65) (layers F.Cu F.Paste F.Mask) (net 1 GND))
  (pad 5 smd rect (at 1.1 0) (size 1.06 0.65) (layers F.Cu F.Paste F.Mask) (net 18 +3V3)))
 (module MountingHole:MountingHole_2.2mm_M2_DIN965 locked (layer F.Cu) (at 205.486 117.475)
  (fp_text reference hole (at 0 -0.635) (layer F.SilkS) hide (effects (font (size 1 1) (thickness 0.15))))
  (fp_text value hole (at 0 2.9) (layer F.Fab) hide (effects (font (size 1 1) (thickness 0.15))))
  (pad 1 np_thru_hole circle (at 0 0) (size 2.2 2.2) (drill 2.2) (layers *.Cu *.Mask)))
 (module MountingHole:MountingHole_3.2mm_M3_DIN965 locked (layer F.Cu) (at 232.791 100.203)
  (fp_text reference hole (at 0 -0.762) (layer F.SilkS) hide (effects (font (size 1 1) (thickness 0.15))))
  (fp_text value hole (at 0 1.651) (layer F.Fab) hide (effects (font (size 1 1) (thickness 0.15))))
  (pad 1 np_thru_hole circle (at 0 0) (size 3.2 3.2) (drill 3.2) (layers *.Cu *.Mask)))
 (gr_line (start 182.499 115.062) (end 207.899 115.062) (layer Edge.Cuts) (width 0.0254))
 (gr_line (start 207.899 140.462) (end 207.899 115.062) (layer Edge.Cuts) (width 0.0254))
 (gr_line (start 182.499 140.462) (end 207.899 140.462) (layer Edge.Cuts) (width 0.0254))
 (gr_line (start 182.499 115.062) (end 182.499 140.462) (layer Edge.Cuts) (width 0.0254))
 (segment (start 156.530754 127.32) (end 157.279 128.068246) (width 0.1524) (layer F.Cu) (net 1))
 (segment (start 155.321 127.32) (end 156.530754 127.32) (width 0.1524) (layer F.Cu) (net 1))
 (segment (start 157.029 129.518246) (end 157.529 129.518246) (width 0.1524) (layer F.Cu) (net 1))
 (segment (start 157.029 128.318246) (end 157.279 128.068246) (width 0.1524) (layer F.Cu) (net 1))
 (segment (start 157.029 129.518246) (end 157.029 128.318246) (width 0.1524) (layer F.Cu) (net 1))
 (segment (start 157.529 128.318246) (end 157.279 128.068246) (width 0.1524) (layer F.Cu) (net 1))
 (segment (start 157.529 129.518246) (end 157.529 128.318246) (width 0.1524) (layer F.Cu) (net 1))
 (segment (start 157.800754 128.59) (end 157.279 128.068246) (width 0.1524) (layer F.Cu) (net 1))
 (segment (start 159.131 128.59) (end 157.800754 128.59) (width 0.1524) (layer F.Cu) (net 1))
 (segment (start 159.131 129.352) (end 159.319 129.54) (width 0.1524) (layer F.Cu) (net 1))
 (segment (start 159.131 128.59) (end 159.131 129.352) (width 0.1524) (layer F.Cu) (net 1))
 (segment (start 191.598 156.083) (end 193.548 156.083) (width 0.1524) (layer F.Cu) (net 1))
 (segment (start 194.998 156.083) (end 193.548 156.083) (width 0.1524) (layer F.Cu) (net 1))
 (segment (start 195.498 156.083) (end 194.998 156.083) (width 0.1524) (layer F.Cu) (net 1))
 (segment (start 156.467246 126.68) (end 156.529 126.618246) (width 0.1524) (layer F.Cu) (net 17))
 (segment (start 155.321 126.68) (end 156.467246 126.68) (width 0.1524) (layer F.Cu) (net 17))
 (via (at 158.623 126.238) (size 0.508) (drill 0.254) (layers F.Cu B.Cu) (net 17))
 (segment (start 159.197 126.238) (end 159.385 126.426) (width 0.1524) (layer F.Cu) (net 17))
 (segment (start 158.623 126.238) (end 159.197 126.238) (width 0.1524) (layer F.Cu) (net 17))
 (via (at 158.623 129.54) (size 0.508) (drill 0.254) (layers F.Cu B.Cu) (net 17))
 (segment (start 158.029 129.518246) (end 158.601246 129.518246) (width 0.1524) (layer F.Cu) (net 17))
 (segment (start 158.601246 129.518246) (end 158.623 129.54) (width 0.1524) (layer F.Cu) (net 17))
 (segment (start 158.623 129.54) (end 158.623 126.238) (width 0.1524) (layer B.Cu) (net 17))
 (via (at 155.448 126.111) (size 0.508) (drill 0.254) (layers F.Cu B.Cu) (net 17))
 (segment (start 155.448 126.68) (end 155.448 126.111) (width 0.1524) (layer F.Cu) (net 17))
 (segment (start 158.496 126.111) (end 158.623 126.238) (width 0.1524) (layer B.Cu) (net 17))
 (segment (start 155.448 126.111) (end 158.496 126.111) (width 0.1524) (layer B.Cu) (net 17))
 (segment (start 157.029 126.618246) (end 157.529 126.618246) (width 0.1524) (layer F.Cu) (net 18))
 (segment (start 160.02 127.62) (end 160.02 127.95) (width 0.1524) (layer F.Cu) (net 18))
 (segment (start 160.02 126.366274) (end 160.02 127.62) (width 0.1524) (layer F.Cu) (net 18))
 (segment (start 157.864447 125.755399) (end 159.409125 125.755399) (width 0.1524) (layer F.Cu) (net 18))
 (segment (start 157.529 126.090846) (end 157.864447 125.755399) (width 0.1524) (layer F.Cu) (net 18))
 (segment (start 159.409125 125.755399) (end 160.02 126.366274) (width 0.1524) (layer F.Cu) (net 18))
 (segment (start 157.529 126.618246) (end 157.529 126.090846) (width 0.1524) (layer F.Cu) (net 18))
 (segment (start 160.02 127.95) (end 159.131 127.95) (width 0.1524) (layer F.Cu) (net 18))
 (segment (start 195.498 156.983) (end 195.498 156.533) (width 0.1524) (layer F.Cu) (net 18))
 (segment (start 159.085 127.066) (end 159.385 127.066) (width 0.1524) (layer F.Cu) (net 19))
 (segment (start 158.251754 127.066) (end 159.085 127.066) (width 0.1524) (layer F.Cu) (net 19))
 (segment (start 158.029 126.843246) (end 158.251754 127.066) (width 0.1524) (layer F.Cu) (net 19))
 (segment (start 158.029 126.618246) (end 158.029 126.843246) (width 0.1524) (layer F.Cu) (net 19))
 (segment (start 160.02 129.479) (end 159.959 129.54) (width 0.1524) (layer F.Cu) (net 20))
 (segment (start 160.02 128.59) (end 160.02 129.479) (width 0.1524) (layer F.Cu) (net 20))
 (segment (start 159.677153 130.121847) (end 156.605201 130.121847) (width 0.1524) (layer F.Cu) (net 20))
 (segment (start 159.959 129.84) (end 159.677153 130.121847) (width 0.1524) (layer F.Cu) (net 20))
 (segment (start 156.529 130.045646) (end 156.529 129.518246) (width 0.1524) (layer F.Cu) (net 20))
 (segment (start 156.605201 130.121847) (end 156.529 130.045646) (width 0.1524) (layer F.Cu) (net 20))
 (segment (start 159.959 129.54) (end 159.959 129.84) (width 0.1524) (layer F.Cu) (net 20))
 (segment (start 201.9735 134.94) (end 203.6735 134.94) (width 0.1524) (layer F.Cu) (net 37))
 (segment (start 203.6735 134.94) (end 205.3735 134.94) (width 0.1524) (layer F.Cu) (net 37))
 (segment (start 205.3735 134.94) (end 207.0735 134.94) (width 0.1524) (layer F.Cu) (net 37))
 (segment (start 183.3245 134.94) (end 185.0245 134.94) (width 0.1524) (layer F.Cu) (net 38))
 (segment (start 185.0245 134.94) (end 186.7245 134.94) (width 0.1524) (layer F.Cu) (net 38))
 (segment (start 187.0245 134.94) (end 188.4245 134.94) (width 0.1524) (layer F.Cu) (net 38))
 (segment (start 186.7245 134.94) (end 187.0245 134.94) (width 0.1524) (layer F.Cu) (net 38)))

